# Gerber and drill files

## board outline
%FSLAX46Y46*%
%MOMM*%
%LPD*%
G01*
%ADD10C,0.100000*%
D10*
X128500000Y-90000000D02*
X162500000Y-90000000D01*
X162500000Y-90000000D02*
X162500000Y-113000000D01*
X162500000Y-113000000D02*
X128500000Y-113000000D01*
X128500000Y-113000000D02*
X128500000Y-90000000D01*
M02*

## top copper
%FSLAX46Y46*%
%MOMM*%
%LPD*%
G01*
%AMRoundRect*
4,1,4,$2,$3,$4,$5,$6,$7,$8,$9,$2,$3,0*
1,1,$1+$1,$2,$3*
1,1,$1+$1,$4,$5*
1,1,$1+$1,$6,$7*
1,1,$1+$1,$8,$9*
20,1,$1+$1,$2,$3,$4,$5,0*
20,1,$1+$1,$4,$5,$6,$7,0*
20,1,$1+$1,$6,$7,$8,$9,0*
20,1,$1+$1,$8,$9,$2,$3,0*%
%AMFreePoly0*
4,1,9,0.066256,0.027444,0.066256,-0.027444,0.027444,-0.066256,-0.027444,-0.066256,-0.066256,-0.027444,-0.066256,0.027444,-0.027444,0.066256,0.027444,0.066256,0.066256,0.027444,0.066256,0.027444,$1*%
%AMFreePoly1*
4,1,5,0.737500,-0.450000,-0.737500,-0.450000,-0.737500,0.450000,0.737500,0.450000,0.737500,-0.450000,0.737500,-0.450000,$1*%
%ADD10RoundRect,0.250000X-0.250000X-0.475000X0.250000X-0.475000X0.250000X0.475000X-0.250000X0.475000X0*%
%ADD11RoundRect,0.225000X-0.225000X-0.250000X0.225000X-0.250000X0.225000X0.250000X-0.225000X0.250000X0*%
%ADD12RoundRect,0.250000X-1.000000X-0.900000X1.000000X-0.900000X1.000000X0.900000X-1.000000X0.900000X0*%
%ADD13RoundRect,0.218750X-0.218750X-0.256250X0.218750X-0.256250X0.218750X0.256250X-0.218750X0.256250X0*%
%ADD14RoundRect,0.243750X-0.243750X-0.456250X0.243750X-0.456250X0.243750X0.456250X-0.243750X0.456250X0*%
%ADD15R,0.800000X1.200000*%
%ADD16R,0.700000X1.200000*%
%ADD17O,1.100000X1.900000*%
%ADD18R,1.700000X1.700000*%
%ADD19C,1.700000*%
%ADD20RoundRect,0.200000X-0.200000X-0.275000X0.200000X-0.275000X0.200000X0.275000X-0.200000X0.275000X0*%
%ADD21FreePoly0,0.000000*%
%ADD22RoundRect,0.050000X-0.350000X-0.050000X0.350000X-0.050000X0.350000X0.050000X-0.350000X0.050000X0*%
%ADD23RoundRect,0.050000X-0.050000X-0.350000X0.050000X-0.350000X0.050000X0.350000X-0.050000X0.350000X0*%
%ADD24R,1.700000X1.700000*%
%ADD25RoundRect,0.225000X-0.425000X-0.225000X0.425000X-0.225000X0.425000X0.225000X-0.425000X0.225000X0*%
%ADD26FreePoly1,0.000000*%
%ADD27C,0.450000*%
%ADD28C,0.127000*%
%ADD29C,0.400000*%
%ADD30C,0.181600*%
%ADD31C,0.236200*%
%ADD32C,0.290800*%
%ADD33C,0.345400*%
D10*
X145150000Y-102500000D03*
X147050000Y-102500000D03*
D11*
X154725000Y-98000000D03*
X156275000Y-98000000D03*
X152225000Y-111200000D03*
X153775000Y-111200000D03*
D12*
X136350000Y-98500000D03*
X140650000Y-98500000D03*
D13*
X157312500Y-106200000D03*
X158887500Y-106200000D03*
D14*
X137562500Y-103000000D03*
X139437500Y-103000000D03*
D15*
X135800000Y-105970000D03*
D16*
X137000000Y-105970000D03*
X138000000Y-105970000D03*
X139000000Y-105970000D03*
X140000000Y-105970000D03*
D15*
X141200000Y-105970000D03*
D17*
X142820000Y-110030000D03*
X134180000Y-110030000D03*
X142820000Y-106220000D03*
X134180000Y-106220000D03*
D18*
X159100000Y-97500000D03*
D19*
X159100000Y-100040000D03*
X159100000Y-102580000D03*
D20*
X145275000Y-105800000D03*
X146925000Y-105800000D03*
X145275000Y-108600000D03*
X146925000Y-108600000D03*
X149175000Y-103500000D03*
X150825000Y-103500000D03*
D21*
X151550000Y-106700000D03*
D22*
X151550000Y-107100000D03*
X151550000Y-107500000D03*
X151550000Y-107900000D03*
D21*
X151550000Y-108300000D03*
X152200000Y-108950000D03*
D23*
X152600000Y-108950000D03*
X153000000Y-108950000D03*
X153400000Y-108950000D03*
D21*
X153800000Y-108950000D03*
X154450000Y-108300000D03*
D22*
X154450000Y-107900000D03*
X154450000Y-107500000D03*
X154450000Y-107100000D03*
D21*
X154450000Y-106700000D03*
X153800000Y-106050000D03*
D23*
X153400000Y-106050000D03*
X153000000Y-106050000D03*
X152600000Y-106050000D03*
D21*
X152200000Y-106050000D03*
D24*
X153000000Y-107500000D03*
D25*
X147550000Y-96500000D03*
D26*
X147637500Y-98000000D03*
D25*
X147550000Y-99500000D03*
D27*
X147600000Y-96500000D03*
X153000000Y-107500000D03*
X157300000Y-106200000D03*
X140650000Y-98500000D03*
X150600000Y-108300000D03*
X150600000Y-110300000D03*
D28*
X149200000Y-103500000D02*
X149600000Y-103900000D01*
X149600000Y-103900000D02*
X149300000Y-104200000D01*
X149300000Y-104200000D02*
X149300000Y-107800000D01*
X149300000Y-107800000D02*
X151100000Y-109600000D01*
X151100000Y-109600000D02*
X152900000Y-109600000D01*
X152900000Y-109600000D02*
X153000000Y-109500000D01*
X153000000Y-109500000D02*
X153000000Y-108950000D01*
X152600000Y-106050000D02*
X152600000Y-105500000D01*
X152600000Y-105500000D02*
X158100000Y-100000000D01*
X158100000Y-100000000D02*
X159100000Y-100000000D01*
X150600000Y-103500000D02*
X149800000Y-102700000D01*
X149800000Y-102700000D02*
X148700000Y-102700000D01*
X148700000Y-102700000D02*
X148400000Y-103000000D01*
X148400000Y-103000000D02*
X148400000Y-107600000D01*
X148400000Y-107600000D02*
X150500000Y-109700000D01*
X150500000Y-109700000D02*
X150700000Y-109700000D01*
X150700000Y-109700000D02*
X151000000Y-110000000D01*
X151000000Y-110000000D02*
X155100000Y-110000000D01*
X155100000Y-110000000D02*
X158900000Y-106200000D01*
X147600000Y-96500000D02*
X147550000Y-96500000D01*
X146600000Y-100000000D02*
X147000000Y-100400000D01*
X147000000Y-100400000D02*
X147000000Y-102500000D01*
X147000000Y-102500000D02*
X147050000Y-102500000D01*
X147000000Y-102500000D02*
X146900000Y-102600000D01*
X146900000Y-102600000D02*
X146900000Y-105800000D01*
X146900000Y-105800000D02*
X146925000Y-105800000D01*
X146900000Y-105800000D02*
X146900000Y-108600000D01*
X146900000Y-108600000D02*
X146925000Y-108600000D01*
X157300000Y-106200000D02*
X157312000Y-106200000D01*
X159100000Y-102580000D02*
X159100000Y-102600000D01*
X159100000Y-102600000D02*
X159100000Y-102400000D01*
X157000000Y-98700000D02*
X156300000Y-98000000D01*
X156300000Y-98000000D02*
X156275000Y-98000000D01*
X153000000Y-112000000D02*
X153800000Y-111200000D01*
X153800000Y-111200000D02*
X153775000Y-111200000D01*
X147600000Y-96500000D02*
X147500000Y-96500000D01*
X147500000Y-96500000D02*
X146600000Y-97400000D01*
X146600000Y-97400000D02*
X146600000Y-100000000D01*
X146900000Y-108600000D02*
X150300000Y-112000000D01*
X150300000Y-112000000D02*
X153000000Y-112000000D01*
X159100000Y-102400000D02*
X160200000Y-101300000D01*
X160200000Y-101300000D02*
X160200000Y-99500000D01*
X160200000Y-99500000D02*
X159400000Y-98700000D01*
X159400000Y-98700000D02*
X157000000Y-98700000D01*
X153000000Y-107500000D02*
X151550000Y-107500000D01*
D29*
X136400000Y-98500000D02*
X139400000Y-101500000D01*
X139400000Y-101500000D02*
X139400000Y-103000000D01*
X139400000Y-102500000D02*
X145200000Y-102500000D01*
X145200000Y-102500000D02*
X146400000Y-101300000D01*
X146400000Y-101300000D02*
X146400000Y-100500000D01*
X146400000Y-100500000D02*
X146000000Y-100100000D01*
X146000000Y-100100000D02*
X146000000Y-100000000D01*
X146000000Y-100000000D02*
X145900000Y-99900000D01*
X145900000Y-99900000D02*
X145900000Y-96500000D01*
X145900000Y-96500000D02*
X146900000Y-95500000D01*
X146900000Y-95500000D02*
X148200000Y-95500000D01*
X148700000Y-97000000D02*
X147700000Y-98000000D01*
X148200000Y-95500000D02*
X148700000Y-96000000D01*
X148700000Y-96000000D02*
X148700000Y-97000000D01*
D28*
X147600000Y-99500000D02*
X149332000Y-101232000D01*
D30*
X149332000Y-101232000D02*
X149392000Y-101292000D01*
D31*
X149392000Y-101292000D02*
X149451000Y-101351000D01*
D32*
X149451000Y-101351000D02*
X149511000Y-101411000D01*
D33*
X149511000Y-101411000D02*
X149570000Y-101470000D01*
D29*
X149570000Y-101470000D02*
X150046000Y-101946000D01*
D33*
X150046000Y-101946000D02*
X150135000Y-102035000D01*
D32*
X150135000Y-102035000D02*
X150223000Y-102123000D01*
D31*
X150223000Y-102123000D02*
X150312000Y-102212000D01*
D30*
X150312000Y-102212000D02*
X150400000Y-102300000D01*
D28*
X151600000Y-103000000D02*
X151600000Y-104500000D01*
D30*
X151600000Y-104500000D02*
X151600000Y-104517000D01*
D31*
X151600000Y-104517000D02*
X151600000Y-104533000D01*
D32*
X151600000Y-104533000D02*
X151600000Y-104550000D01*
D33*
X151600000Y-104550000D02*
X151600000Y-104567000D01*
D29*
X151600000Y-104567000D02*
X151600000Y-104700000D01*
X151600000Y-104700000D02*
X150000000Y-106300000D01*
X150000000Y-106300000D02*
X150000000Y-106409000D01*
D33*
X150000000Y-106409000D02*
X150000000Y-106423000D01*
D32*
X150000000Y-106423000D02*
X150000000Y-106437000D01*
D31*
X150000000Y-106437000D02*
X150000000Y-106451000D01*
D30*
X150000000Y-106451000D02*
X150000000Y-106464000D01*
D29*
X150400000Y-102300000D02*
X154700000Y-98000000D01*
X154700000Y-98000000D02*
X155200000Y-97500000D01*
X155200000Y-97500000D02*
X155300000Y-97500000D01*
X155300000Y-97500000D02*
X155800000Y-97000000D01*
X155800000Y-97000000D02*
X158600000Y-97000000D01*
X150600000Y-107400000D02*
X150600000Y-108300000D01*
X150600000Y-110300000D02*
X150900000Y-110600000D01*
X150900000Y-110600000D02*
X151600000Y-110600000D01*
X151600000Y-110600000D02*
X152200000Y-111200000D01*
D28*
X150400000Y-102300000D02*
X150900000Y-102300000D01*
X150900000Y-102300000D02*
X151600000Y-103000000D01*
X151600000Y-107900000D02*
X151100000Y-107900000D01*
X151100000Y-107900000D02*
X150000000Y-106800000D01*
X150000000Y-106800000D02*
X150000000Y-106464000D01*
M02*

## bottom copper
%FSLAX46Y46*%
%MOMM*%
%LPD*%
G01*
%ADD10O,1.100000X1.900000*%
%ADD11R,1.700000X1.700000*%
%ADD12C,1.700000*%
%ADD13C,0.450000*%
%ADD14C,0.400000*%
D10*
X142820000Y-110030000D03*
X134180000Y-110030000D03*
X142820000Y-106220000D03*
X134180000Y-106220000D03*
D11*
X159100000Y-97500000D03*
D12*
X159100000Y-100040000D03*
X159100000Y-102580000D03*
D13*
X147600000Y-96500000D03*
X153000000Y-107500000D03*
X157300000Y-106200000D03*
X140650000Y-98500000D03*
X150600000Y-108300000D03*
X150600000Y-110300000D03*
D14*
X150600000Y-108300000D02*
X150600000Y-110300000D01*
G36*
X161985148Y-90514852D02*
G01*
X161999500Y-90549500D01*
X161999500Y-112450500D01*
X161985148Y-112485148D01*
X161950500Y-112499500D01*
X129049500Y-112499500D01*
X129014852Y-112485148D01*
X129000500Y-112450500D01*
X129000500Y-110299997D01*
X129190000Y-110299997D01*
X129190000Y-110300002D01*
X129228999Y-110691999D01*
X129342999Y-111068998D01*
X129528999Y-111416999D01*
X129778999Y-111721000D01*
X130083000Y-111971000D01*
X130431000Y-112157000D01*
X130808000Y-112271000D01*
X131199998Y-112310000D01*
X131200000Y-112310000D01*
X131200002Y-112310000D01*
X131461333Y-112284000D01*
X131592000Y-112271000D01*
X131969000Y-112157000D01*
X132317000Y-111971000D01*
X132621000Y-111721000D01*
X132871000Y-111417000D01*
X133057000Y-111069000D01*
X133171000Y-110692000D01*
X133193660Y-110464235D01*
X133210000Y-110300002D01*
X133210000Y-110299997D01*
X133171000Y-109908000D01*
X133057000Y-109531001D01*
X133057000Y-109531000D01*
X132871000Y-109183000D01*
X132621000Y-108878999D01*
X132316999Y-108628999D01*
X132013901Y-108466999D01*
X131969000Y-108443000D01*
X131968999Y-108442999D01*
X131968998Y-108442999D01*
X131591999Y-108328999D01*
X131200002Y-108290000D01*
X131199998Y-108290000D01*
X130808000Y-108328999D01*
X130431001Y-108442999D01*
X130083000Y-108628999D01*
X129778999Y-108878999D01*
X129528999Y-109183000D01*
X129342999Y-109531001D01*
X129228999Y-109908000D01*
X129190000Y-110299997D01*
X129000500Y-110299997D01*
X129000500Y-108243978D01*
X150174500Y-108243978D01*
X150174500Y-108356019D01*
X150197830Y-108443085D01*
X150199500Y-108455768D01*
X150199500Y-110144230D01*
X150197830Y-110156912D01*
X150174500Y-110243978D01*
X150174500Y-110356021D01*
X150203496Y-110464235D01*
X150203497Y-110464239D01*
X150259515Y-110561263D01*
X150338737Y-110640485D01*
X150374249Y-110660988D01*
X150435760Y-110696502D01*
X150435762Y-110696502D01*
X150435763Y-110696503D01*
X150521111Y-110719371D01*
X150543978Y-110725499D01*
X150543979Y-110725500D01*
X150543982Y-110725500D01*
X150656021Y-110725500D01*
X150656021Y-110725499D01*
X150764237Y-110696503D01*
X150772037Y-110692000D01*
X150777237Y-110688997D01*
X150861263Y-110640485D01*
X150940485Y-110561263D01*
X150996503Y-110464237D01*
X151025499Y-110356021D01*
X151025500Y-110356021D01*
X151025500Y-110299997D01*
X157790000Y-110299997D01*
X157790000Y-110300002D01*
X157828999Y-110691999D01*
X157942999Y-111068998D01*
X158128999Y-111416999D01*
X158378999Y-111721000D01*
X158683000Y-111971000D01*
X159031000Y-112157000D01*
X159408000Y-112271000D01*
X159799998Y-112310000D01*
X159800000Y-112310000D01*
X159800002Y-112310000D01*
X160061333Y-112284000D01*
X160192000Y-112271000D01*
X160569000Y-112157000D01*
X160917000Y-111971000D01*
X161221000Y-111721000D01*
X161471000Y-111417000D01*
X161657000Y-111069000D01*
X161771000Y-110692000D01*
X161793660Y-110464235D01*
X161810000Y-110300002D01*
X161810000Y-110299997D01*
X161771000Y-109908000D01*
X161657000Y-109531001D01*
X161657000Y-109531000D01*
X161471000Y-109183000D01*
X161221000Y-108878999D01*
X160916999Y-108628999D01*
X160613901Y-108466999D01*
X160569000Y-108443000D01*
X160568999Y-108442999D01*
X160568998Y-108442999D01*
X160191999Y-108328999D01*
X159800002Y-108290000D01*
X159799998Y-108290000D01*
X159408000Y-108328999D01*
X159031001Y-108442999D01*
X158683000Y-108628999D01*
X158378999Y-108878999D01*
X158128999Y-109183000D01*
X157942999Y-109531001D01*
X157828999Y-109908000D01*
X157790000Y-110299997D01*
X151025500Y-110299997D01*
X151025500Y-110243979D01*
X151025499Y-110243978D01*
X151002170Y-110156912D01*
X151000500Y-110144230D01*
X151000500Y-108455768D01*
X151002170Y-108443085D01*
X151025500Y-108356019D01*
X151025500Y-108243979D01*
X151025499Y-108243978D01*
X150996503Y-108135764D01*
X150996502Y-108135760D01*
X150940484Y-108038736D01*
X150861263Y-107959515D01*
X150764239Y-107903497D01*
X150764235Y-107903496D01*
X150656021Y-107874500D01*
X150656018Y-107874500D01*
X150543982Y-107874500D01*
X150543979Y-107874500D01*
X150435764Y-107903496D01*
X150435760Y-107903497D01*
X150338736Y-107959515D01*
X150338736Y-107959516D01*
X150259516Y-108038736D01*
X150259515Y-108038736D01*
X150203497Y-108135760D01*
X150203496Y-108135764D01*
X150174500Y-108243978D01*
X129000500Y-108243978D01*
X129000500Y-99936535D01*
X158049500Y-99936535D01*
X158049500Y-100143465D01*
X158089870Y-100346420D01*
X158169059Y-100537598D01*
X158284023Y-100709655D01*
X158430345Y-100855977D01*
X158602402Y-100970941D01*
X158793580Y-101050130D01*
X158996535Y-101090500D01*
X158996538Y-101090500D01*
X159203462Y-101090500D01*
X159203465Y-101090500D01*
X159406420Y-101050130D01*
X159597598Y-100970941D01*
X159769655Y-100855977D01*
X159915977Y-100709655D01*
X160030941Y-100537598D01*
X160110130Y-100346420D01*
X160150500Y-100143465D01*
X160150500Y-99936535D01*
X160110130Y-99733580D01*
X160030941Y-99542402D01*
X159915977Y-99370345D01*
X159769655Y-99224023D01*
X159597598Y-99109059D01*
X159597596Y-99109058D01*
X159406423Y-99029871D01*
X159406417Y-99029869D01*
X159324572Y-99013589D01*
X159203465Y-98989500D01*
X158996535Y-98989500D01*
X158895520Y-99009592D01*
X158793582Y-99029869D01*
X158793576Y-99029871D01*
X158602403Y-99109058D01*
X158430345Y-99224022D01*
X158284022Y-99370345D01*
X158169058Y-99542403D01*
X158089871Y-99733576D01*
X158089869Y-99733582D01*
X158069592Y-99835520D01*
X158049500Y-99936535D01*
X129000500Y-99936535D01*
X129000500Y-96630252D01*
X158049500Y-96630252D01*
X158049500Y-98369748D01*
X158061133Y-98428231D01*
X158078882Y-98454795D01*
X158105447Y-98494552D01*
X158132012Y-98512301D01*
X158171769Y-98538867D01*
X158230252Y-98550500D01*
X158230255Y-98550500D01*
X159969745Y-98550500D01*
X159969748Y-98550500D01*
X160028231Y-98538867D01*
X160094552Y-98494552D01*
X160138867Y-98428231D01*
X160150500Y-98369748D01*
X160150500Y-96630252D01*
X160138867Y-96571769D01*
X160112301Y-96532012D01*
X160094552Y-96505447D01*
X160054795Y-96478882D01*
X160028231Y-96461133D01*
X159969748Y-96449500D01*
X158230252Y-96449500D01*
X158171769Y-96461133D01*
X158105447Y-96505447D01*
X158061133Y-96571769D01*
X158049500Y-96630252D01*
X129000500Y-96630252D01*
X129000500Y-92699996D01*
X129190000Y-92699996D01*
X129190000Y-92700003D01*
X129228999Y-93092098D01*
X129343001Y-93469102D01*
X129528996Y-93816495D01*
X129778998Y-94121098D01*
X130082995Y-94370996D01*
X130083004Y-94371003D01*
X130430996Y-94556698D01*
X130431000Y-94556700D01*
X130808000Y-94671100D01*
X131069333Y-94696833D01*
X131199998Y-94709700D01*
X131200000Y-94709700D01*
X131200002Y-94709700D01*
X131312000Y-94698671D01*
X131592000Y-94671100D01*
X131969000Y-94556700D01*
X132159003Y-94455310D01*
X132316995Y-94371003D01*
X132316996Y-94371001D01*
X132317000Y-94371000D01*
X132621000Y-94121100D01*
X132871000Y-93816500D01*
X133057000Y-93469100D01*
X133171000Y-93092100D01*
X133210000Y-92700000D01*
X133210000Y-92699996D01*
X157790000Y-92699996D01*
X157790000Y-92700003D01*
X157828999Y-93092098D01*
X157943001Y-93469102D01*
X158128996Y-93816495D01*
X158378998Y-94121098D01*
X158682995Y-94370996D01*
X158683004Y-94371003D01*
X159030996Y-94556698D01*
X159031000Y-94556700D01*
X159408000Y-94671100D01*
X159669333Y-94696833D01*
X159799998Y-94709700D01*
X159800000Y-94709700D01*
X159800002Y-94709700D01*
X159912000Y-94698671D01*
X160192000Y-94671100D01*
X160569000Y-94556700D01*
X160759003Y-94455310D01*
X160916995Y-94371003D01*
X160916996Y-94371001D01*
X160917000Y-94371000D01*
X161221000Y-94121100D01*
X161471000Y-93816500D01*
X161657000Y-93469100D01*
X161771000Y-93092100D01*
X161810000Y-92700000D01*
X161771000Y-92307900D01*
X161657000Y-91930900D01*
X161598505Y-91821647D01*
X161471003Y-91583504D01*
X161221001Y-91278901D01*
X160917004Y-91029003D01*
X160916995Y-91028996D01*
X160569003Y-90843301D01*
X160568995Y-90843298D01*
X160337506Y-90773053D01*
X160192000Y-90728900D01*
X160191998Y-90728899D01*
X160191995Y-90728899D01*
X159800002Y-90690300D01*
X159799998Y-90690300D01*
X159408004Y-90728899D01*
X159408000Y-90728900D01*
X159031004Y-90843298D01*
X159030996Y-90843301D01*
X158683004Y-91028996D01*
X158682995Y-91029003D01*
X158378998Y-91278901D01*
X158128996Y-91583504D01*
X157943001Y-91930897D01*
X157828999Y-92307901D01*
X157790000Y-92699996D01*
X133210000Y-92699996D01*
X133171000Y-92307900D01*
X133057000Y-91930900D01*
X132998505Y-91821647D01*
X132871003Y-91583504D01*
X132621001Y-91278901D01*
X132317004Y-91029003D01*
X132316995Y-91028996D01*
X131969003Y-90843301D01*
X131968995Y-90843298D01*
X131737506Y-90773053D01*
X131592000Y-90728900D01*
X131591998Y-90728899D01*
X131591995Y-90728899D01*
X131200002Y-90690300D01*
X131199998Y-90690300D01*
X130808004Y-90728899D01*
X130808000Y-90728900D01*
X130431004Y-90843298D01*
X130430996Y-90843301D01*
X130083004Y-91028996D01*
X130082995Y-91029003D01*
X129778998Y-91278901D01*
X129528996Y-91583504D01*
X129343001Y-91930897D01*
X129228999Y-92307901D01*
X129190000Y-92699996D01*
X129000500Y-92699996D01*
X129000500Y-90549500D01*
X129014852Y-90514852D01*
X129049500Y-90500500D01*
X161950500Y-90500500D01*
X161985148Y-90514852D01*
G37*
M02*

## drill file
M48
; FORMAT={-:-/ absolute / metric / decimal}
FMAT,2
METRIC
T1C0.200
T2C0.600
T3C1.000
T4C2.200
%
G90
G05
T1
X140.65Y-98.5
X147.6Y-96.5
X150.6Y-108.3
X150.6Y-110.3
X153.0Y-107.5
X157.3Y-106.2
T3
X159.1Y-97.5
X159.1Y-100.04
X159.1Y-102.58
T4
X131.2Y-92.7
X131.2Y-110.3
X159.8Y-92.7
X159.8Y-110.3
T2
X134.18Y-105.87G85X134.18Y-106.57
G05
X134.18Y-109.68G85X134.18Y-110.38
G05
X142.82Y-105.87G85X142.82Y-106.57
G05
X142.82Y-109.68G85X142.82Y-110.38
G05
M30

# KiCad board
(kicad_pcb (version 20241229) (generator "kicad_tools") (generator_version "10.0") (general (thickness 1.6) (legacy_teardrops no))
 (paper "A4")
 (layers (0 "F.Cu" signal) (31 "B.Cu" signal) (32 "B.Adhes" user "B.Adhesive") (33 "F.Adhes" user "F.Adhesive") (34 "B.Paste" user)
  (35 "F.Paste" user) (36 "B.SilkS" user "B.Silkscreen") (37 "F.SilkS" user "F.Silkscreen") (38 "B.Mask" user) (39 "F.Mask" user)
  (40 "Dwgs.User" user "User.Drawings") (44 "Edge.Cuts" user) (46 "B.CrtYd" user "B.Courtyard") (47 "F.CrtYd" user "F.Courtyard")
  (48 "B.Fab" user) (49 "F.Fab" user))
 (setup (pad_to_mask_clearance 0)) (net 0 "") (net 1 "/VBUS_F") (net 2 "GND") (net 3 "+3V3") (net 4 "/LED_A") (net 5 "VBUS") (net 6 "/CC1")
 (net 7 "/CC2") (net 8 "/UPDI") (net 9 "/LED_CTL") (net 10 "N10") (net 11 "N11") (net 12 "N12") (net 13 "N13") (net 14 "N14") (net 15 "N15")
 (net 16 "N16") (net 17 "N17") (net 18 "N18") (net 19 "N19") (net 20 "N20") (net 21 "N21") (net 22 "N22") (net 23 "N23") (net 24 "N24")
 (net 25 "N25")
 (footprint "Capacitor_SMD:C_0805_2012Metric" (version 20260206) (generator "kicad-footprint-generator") (layer "F.Cu") (at 146.1 102.5)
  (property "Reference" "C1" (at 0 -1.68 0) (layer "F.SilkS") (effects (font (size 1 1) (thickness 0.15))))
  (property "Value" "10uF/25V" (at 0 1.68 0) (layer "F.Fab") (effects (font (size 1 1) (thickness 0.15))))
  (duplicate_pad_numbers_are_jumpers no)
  (pad "1" smd roundrect (at -0.95 0) (size 1 1.45) (layers "F.Cu" "F.Mask" "F.Paste") (roundrect_rratio 0.25) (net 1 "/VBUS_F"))
  (pad "2" smd roundrect (at 0.95 0) (size 1 1.45) (layers "F.Cu" "F.Mask" "F.Paste") (roundrect_rratio 0.25) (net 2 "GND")))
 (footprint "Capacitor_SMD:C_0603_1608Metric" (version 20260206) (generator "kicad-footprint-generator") (layer "F.Cu") (at 155.5 98)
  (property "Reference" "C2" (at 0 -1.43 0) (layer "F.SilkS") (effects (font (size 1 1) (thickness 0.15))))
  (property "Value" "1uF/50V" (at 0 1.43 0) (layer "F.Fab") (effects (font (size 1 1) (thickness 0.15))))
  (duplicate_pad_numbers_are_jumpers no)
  (pad "1" smd roundrect (at -0.775 0) (size 0.9 0.95) (layers "F.Cu" "F.Mask" "F.Paste") (roundrect_rratio 0.25) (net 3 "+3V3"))
  (pad "2" smd roundrect (at 0.775 0) (size 0.9 0.95) (layers "F.Cu" "F.Mask" "F.Paste") (roundrect_rratio 0.25) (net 2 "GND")))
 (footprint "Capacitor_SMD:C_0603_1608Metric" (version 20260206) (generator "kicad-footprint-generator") (layer "F.Cu") (at 153 111.2)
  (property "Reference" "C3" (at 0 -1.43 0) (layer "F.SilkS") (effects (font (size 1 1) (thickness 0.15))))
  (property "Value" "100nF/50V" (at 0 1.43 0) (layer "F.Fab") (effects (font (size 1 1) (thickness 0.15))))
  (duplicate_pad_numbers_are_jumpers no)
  (pad "1" smd roundrect (at -0.775 0) (size 0.9 0.95) (layers "F.Cu" "F.Mask" "F.Paste") (roundrect_rratio 0.25) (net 3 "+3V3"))
  (pad "2" smd roundrect (at 0.775 0) (size 0.9 0.95) (layers "F.Cu" "F.Mask" "F.Paste") (roundrect_rratio 0.25) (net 2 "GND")))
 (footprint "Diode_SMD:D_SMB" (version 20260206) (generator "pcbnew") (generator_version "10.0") (layer "F.Cu") (at 138.5 98.5)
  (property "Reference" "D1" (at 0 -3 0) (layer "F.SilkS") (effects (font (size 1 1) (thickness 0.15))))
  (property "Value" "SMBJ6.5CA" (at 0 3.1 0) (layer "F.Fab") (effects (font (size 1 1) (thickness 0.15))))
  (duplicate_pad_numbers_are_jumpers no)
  (pad "1" smd roundrect (at -2.15 0) (size 2.5 2.3) (layers "F.Cu" "F.Mask" "F.Paste") (roundrect_rratio 0.1086956522) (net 1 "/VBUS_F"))
  (pad "2" smd roundrect (at 2.15 0) (size 2.5 2.3) (layers "F.Cu" "F.Mask" "F.Paste") (roundrect_rratio 0.1086956522) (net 2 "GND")))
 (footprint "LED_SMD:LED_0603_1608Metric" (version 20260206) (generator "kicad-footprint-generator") (layer "F.Cu") (at 158.1 106.2)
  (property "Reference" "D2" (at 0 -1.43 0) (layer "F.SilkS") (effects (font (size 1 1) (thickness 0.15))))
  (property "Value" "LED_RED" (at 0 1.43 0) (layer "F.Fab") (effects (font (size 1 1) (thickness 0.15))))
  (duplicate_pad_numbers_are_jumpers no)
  (pad "1" smd roundrect (at -0.7875 0) (size 0.875 0.95) (layers "F.Cu" "F.Mask" "F.Paste") (roundrect_rratio 0.25) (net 2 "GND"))
  (pad "2" smd roundrect (at 0.7875 0) (size 0.875 0.95) (layers "F.Cu" "F.Mask" "F.Paste") (roundrect_rratio 0.25) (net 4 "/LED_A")))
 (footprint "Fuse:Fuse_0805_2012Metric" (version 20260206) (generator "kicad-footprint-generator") (layer "F.Cu") (at 138.5 103)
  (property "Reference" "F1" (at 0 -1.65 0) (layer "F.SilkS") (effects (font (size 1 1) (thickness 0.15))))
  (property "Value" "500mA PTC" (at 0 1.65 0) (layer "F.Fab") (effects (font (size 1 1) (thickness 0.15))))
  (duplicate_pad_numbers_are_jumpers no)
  (pad "1" smd roundrect (at -0.9375 0) (size 0.975 1.4) (layers "F.Cu" "F.Mask" "F.Paste") (roundrect_rratio 0.25) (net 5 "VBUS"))
  (pad "2" smd roundrect (at 0.9375 0) (size 0.975 1.4) (layers "F.Cu" "F.Mask" "F.Paste") (roundrect_rratio 0.25) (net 1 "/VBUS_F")))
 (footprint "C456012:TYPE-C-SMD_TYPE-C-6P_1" (layer "F.Cu") (at 138.5 108)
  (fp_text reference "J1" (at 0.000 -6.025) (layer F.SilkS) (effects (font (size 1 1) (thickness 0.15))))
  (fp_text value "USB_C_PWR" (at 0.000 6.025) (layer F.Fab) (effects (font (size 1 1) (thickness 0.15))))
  (pad B12 smd rect (at -2.70 -2.03 0.00) (size 0.800 1.200) (layers F.Cu F.Paste F.Mask) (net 2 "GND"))
  (pad B9 smd rect (at -1.50 -2.03 0.00) (size 0.700 1.200) (layers F.Cu F.Paste F.Mask) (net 5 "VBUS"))
  (pad A5 smd rect (at -0.50 -2.03 0.00) (size 0.700 1.200) (layers F.Cu F.Paste F.Mask) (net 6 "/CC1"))
  (pad B5 smd rect (at 0.50 -2.03 0.00) (size 0.700 1.200) (layers F.Cu F.Paste F.Mask) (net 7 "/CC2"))
  (pad A9 smd rect (at 1.50 -2.03 0.00) (size 0.700 1.200) (layers F.Cu F.Paste F.Mask) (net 5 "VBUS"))
  (pad A12 smd rect (at 2.70 -2.03 0.00) (size 0.800 1.200) (layers F.Cu F.Paste F.Mask) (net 2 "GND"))
  (pad 7 thru_hole oval (at 4.32 2.03 0.00) (size 1.100 1.900) (layers *.Cu *.Mask) (drill oval 0.599998 1.299997) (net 2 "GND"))
  (pad 7 thru_hole oval (at -4.32 2.03 0.00) (size 1.100 1.900) (layers *.Cu *.Mask) (drill oval 0.599998 1.299997) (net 2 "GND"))
  (pad 7 thru_hole oval (at 4.32 -1.78 0.00) (size 1.100 1.900) (layers *.Cu *.Mask) (drill oval 0.599998 1.299997) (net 2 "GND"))
  (pad 7 thru_hole oval (at -4.32 -1.78 0.00) (size 1.100 1.900) (layers *.Cu *.Mask) (drill oval 0.599998 1.299997) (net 2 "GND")))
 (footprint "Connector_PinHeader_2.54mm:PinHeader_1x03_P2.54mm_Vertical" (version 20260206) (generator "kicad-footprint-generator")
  (layer "F.Cu") (at 159.1 97.5)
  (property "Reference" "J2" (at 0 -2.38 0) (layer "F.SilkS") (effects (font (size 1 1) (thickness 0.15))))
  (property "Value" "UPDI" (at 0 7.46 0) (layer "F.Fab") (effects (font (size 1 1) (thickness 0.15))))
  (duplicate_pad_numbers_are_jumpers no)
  (pad "1" thru_hole rect (at 0 0) (size 1.7 1.7) (drill 1) (layers "*.Cu" "*.Mask") (remove_unused_layers no) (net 3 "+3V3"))
  (pad "2" thru_hole circle (at 0 2.54) (size 1.7 1.7) (drill 1) (layers "*.Cu" "*.Mask") (remove_unused_layers no) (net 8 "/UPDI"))
  (pad "3" thru_hole circle (at 0 5.08) (size 1.7 1.7) (drill 1) (layers "*.Cu" "*.Mask") (remove_unused_layers no) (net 2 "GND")))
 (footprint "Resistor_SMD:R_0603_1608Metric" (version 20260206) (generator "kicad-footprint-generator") (layer "F.Cu") (at 146.1 105.8)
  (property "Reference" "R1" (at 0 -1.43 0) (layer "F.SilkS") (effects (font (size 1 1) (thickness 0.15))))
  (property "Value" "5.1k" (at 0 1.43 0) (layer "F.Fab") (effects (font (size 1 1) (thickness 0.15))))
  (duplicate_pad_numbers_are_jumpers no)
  (pad "1" smd roundrect (at -0.825 0) (size 0.8 0.95) (layers "F.Cu" "F.Mask" "F.Paste") (roundrect_rratio 0.25) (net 6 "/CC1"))
  (pad "2" smd roundrect (at 0.825 0) (size 0.8 0.95) (layers "F.Cu" "F.Mask" "F.Paste") (roundrect_rratio 0.25) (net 2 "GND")))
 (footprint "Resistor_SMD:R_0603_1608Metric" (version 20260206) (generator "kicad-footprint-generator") (layer "F.Cu") (at 146.1 108.6)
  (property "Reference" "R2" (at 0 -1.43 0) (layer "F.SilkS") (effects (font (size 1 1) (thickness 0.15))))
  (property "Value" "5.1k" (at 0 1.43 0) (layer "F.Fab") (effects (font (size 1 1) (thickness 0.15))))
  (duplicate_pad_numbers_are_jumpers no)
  (pad "1" smd roundrect (at -0.825 0) (size 0.8 0.95) (layers "F.Cu" "F.Mask" "F.Paste") (roundrect_rratio 0.25) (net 7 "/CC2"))
  (pad "2" smd roundrect (at 0.825 0) (size 0.8 0.95) (layers "F.Cu" "F.Mask" "F.Paste") (roundrect_rratio 0.25) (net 2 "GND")))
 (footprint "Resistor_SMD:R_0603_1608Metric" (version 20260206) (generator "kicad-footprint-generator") (layer "F.Cu") (at 150 103.5)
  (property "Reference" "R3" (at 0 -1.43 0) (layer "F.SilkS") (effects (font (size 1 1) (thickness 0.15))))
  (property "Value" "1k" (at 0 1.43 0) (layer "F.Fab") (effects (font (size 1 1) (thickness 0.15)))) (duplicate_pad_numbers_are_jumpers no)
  (pad "1" smd roundrect (at -0.825 0) (size 0.8 0.95) (layers "F.Cu" "F.Mask" "F.Paste") (roundrect_rratio 0.25) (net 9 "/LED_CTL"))
  (pad "2" smd roundrect (at 0.825 0) (size 0.8 0.95) (layers "F.Cu" "F.Mask" "F.Paste") (roundrect_rratio 0.25) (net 4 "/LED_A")))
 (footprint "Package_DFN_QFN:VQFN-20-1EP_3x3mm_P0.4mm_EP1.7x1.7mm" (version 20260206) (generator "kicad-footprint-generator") (layer "F.Cu")
  (at 153 107.5)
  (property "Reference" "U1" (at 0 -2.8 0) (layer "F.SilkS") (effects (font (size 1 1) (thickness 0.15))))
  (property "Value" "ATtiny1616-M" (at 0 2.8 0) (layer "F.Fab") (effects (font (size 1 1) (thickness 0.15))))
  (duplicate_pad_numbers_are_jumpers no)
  (pad "" smd roundrect (at -0.425 -0.425) (size 0.69 0.69) (layers "F.Paste") (roundrect_rratio 0.25))
  (pad "" smd roundrect (at -0.425 0.425) (size 0.69 0.69) (layers "F.Paste") (roundrect_rratio 0.25))
  (pad "" smd roundrect (at 0.425 -0.425) (size 0.69 0.69) (layers "F.Paste") (roundrect_rratio 0.25))
  (pad "" smd roundrect (at 0.425 0.425) (size 0.69 0.69) (layers "F.Paste") (roundrect_rratio 0.25))
  (pad "1" smd custom (at -1.45 -0.8) (size 0.143431 0.143431) (layers "F.Cu" "F.Mask" "F.Paste")
   (options (clearance outline) (anchor circle)) (primitives) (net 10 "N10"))
  (pad "2" smd roundrect (at -1.45 -0.4) (size 0.8 0.2) (layers "F.Cu" "F.Mask" "F.Paste") (roundrect_rratio 0.25) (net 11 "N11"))
  (pad "3" smd roundrect (at -1.45 0) (size 0.8 0.2) (layers "F.Cu" "F.Mask" "F.Paste") (roundrect_rratio 0.25) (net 2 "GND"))
  (pad "4" smd roundrect (at -1.45 0.4) (size 0.8 0.2) (layers "F.Cu" "F.Mask" "F.Paste") (roundrect_rratio 0.25) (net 3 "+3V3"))
  (pad "5" smd custom (at -1.45 0.8) (size 0.143431 0.143431) (layers "F.Cu" "F.Mask" "F.Paste")
   (options (clearance outline) (anchor circle)) (primitives) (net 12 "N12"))
  (pad "6" smd custom (at -0.8 1.45) (size 0.143431 0.143431) (layers "F.Cu" "F.Mask" "F.Paste")
   (options (clearance outline) (anchor circle)) (primitives) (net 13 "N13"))
  (pad "7" smd roundrect (at -0.4 1.45) (size 0.2 0.8) (layers "F.Cu" "F.Mask" "F.Paste") (roundrect_rratio 0.25) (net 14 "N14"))
  (pad "8" smd roundrect (at 0 1.45) (size 0.2 0.8) (layers "F.Cu" "F.Mask" "F.Paste") (roundrect_rratio 0.25) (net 9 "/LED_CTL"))
  (pad "9" smd roundrect (at 0.4 1.45) (size 0.2 0.8) (layers "F.Cu" "F.Mask" "F.Paste") (roundrect_rratio 0.25) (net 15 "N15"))
  (pad "10" smd custom (at 0.8 1.45) (size 0.143431 0.143431) (layers "F.Cu" "F.Mask" "F.Paste")
   (options (clearance outline) (anchor circle)) (primitives) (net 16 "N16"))
  (pad "11" smd custom (at 1.45 0.8) (size 0.143431 0.143431) (layers "F.Cu" "F.Mask" "F.Paste")
   (options (clearance outline) (anchor circle)) (primitives) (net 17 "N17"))
  (pad "12" smd roundrect (at 1.45 0.4) (size 0.8 0.2) (layers "F.Cu" "F.Mask" "F.Paste") (roundrect_rratio 0.25) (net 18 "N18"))
  (pad "13" smd roundrect (at 1.45 0) (size 0.8 0.2) (layers "F.Cu" "F.Mask" "F.Paste") (roundrect_rratio 0.25) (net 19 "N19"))
  (pad "14" smd roundrect (at 1.45 -0.4) (size 0.8 0.2) (layers "F.Cu" "F.Mask" "F.Paste") (roundrect_rratio 0.25) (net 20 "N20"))
  (pad "15" smd custom (at 1.45 -0.8) (size 0.143431 0.143431) (layers "F.Cu" "F.Mask" "F.Paste")
   (options (clearance outline) (anchor circle)) (primitives) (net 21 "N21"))
  (pad "16" smd custom (at 0.8 -1.45) (size 0.143431 0.143431) (layers "F.Cu" "F.Mask" "F.Paste")
   (options (clearance outline) (anchor circle)) (primitives) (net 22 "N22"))
  (pad "17" smd roundrect (at 0.4 -1.45) (size 0.2 0.8) (layers "F.Cu" "F.Mask" "F.Paste") (roundrect_rratio 0.25) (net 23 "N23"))
  (pad "18" smd roundrect (at 0 -1.45) (size 0.2 0.8) (layers "F.Cu" "F.Mask" "F.Paste") (roundrect_rratio 0.25) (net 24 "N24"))
  (pad "19" smd roundrect (at -0.4 -1.45) (size 0.2 0.8) (layers "F.Cu" "F.Mask" "F.Paste") (roundrect_rratio 0.25) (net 8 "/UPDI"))
  (pad "20" smd custom (at -0.8 -1.45) (size 0.143431 0.143431) (layers "F.Cu" "F.Mask" "F.Paste")
   (options (clearance outline) (anchor circle)) (primitives) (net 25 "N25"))
  (pad "21" smd rect (at 0 0) (size 1.7 1.7) (layers "F.Cu" "F.Mask") (zone_connect 2) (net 2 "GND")))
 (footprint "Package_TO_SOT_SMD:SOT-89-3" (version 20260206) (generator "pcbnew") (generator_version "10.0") (layer "F.Cu") (at 149.5 98)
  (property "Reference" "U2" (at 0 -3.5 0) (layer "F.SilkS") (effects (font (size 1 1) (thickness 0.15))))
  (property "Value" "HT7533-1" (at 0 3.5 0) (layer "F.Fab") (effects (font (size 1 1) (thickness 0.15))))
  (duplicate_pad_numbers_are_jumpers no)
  (pad "1" smd roundrect (at -1.95 -1.5) (size 1.3 0.9) (layers "F.Cu" "F.Mask" "F.Paste") (roundrect_rratio 0.25) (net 2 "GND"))
  (pad "2" smd custom (at -1.8625 0) (size 1.475 0.9) (layers "F.Cu" "F.Mask" "F.Paste") (zone_connect 2) (thermal_bridge_angle 45)
   (options (clearance outline) (anchor rect)) (primitives) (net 1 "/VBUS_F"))
  (pad "3" smd roundrect (at -1.95 1.5) (size 1.3 0.9) (layers "F.Cu" "F.Mask" "F.Paste") (roundrect_rratio 0.25) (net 3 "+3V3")))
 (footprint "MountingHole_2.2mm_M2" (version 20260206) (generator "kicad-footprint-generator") (layer "F.Cu") (at 131.2 92.7)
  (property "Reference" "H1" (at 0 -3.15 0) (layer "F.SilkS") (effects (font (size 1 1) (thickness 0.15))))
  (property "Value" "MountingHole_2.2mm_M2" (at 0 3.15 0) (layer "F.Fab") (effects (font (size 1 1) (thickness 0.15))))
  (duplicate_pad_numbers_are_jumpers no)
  (pad "" np_thru_hole circle (at 0 0) (size 2.2 2.2) (drill 2.2) (layers "*.Cu" "*.Mask")))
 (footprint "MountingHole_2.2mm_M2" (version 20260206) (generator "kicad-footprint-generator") (layer "F.Cu") (at 159.8 92.7)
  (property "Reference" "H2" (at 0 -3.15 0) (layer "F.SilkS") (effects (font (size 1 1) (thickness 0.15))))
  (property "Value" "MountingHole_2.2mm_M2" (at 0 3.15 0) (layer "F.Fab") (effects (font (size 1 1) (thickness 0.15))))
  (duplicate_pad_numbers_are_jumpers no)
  (pad "" np_thru_hole circle (at 0 0) (size 2.2 2.2) (drill 2.2) (layers "*.Cu" "*.Mask")))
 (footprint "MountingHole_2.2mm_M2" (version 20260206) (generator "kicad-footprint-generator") (layer "F.Cu") (at 131.2 110.3)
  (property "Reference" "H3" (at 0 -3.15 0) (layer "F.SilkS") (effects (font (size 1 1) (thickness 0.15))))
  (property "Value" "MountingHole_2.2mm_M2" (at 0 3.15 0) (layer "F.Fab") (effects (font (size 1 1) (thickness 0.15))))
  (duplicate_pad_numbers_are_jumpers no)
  (pad "" np_thru_hole circle (at 0 0) (size 2.2 2.2) (drill 2.2) (layers "*.Cu" "*.Mask")))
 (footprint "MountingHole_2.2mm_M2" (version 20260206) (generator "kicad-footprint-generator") (layer "F.Cu") (at 159.8 110.3)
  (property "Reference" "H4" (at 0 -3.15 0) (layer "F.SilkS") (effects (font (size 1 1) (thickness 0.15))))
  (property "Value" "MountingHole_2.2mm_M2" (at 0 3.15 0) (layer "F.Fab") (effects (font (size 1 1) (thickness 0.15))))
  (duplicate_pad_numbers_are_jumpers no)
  (pad "" np_thru_hole circle (at 0 0) (size 2.2 2.2) (drill 2.2) (layers "*.Cu" "*.Mask")))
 (gr_line (start 128.5 90) (end 162.5 90) (stroke (width 0.1) (type default)) (layer "Edge.Cuts"))
 (gr_line (start 162.5 90) (end 162.5 113) (stroke (width 0.1) (type default)) (layer "Edge.Cuts"))
 (gr_line (start 162.5 113) (end 128.5 113) (stroke (width 0.1) (type default)) (layer "Edge.Cuts"))
 (gr_line (start 128.5 113) (end 128.5 90) (stroke (width 0.1) (type default)) (layer "Edge.Cuts"))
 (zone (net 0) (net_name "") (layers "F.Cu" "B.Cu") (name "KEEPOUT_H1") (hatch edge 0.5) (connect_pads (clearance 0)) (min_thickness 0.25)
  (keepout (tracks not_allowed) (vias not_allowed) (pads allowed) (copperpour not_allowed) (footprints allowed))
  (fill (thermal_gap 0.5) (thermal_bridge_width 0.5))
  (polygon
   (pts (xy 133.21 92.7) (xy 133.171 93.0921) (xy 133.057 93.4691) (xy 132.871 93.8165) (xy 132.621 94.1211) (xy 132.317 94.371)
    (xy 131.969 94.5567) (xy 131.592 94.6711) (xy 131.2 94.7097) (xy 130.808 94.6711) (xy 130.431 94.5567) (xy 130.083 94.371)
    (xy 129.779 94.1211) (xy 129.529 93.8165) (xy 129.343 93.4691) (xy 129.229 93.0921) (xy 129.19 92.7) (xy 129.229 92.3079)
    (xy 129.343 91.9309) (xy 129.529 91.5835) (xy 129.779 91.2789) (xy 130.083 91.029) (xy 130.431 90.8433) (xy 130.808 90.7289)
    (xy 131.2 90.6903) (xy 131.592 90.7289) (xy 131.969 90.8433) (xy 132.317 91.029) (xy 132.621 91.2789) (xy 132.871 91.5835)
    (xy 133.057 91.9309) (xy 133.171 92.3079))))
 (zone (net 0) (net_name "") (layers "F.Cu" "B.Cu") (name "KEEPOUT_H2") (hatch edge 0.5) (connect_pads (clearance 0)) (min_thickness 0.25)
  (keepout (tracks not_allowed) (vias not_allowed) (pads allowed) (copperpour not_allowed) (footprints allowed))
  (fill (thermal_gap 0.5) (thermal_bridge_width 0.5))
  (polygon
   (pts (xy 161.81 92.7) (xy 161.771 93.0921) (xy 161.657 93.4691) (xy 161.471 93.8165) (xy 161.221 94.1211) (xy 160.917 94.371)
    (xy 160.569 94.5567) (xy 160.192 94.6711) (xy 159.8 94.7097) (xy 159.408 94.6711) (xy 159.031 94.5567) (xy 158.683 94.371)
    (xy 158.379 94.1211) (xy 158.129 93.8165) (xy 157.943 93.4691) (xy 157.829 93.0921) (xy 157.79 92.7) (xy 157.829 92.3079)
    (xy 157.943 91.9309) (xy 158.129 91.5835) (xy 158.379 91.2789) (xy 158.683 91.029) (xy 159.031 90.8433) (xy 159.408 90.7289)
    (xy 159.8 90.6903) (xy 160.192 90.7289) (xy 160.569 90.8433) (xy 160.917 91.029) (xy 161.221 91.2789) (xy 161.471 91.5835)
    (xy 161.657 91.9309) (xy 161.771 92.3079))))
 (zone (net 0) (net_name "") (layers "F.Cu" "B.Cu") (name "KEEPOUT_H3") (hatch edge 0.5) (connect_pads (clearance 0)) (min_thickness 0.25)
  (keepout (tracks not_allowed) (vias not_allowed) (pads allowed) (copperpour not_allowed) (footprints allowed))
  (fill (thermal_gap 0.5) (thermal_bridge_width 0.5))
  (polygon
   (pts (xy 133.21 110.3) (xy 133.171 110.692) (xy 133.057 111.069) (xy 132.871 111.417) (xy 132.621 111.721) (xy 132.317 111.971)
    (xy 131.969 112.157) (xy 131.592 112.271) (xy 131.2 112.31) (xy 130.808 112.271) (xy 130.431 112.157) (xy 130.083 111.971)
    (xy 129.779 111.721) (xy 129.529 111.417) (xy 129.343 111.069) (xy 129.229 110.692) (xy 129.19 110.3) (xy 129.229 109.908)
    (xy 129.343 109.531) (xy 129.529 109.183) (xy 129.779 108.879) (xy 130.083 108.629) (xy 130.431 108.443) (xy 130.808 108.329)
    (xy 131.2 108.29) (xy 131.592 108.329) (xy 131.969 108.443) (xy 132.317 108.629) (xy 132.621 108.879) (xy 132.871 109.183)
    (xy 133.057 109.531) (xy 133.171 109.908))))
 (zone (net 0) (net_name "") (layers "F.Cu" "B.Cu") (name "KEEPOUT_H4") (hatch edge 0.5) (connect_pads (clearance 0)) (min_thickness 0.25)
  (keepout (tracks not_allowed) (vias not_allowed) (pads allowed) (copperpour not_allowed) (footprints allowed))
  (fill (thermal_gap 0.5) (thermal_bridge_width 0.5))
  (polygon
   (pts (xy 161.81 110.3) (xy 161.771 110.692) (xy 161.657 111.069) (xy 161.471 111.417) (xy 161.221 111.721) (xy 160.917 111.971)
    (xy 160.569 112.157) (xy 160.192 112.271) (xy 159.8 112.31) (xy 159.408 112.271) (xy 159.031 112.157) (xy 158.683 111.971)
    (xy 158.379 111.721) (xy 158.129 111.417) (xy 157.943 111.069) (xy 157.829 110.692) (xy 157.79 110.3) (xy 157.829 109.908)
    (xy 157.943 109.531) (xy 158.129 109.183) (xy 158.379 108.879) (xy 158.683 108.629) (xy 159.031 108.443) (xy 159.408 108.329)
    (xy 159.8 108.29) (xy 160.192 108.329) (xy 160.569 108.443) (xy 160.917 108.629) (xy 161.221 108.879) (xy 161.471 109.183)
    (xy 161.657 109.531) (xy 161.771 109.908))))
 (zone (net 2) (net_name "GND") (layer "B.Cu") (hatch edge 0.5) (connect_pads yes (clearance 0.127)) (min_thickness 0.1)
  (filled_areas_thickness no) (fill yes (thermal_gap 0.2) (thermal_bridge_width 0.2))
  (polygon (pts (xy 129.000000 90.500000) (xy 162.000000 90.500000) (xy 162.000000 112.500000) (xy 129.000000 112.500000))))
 (segment (start 149.2 103.5) (end 149.6 103.9) (width 0.127) (layer "F.Cu") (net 9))
 (segment (start 149.6 103.9) (end 149.3 104.2) (width 0.127) (layer "F.Cu") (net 9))
 (segment (start 149.3 104.2) (end 149.3 107.8) (width 0.127) (layer "F.Cu") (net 9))
 (segment (start 149.3 107.8) (end 151.1 109.6) (width 0.127) (layer "F.Cu") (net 9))
 (segment (start 151.1 109.6) (end 152.9 109.6) (width 0.127) (layer "F.Cu") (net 9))
 (segment (start 152.9 109.6) (end 153 109.5) (width 0.127) (layer "F.Cu") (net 9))
 (segment (start 153 109.5) (end 153 108.95) (width 0.127) (layer "F.Cu") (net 9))
 (segment (start 152.6 106.05) (end 152.6 105.5) (width 0.127) (layer "F.Cu") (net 8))
 (segment (start 152.6 105.5) (end 158.1 100) (width 0.127) (layer "F.Cu") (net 8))
 (segment (start 158.1 100) (end 159.1 100) (width 0.127) (layer "F.Cu") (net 8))
 (segment (start 150.6 103.5) (end 149.8 102.7) (width 0.127) (layer "F.Cu") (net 4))
 (segment (start 149.8 102.7) (end 148.7 102.7) (width 0.127) (layer "F.Cu") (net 4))
 (segment (start 148.7 102.7) (end 148.4 103) (width 0.127) (layer "F.Cu") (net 4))
 (segment (start 148.4 103) (end 148.4 107.6) (width 0.127) (layer "F.Cu") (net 4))
 (segment (start 148.4 107.6) (end 150.5 109.7) (width 0.127) (layer "F.Cu") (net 4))
 (segment (start 150.5 109.7) (end 150.7 109.7) (width 0.127) (layer "F.Cu") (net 4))
 (segment (start 150.7 109.7) (end 151 110) (width 0.127) (layer "F.Cu") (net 4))
 (segment (start 151 110) (end 155.1 110) (width 0.127) (layer "F.Cu") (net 4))
 (segment (start 155.1 110) (end 158.9 106.2) (width 0.127) (layer "F.Cu") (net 4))
 (segment (start 147.6 96.5) (end 147.55 96.5) (width 0.127) (layer "F.Cu") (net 2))
 (segment (start 146.6 100) (end 147 100.4) (width 0.127) (layer "F.Cu") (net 2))
 (segment (start 147 100.4) (end 147 102.5) (width 0.127) (layer "F.Cu") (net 2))
 (segment (start 147 102.5) (end 147.05 102.5) (width 0.127) (layer "F.Cu") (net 2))
 (segment (start 147 102.5) (end 146.9 102.6) (width 0.127) (layer "F.Cu") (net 2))
 (segment (start 146.9 102.6) (end 146.9 105.8) (width 0.127) (layer "F.Cu") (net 2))
 (segment (start 146.9 105.8) (end 146.925 105.8) (width 0.127) (layer "F.Cu") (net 2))
 (segment (start 146.9 105.8) (end 146.9 108.6) (width 0.127) (layer "F.Cu") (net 2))
 (segment (start 146.9 108.6) (end 146.925 108.6) (width 0.127) (layer "F.Cu") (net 2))
 (segment (start 157.3 106.2) (end 157.312 106.2) (width 0.127) (layer "F.Cu") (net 2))
 (segment (start 159.1 102.58) (end 159.1 102.6) (width 0.127) (layer "F.Cu") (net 2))
 (segment (start 159.1 102.6) (end 159.1 102.4) (width 0.127) (layer "F.Cu") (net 2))
 (segment (start 157 98.7) (end 156.3 98) (width 0.127) (layer "F.Cu") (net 2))
 (segment (start 156.3 98) (end 156.275 98) (width 0.127) (layer "F.Cu") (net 2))
 (segment (start 153 112) (end 153.8 111.2) (width 0.127) (layer "F.Cu") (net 2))
 (segment (start 153.8 111.2) (end 153.775 111.2) (width 0.127) (layer "F.Cu") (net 2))
 (segment (start 147.6 96.5) (end 147.5 96.5) (width 0.127) (layer "F.Cu") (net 2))
 (segment (start 147.5 96.5) (end 146.6 97.4) (width 0.127) (layer "F.Cu") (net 2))
 (segment (start 146.6 97.4) (end 146.6 100) (width 0.127) (layer "F.Cu") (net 2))
 (segment (start 146.9 108.6) (end 150.3 112) (width 0.127) (layer "F.Cu") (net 2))
 (segment (start 150.3 112) (end 153 112) (width 0.127) (layer "F.Cu") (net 2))
 (segment (start 159.1 102.4) (end 160.2 101.3) (width 0.127) (layer "F.Cu") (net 2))
 (segment (start 160.2 101.3) (end 160.2 99.5) (width 0.127) (layer "F.Cu") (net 2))
 (segment (start 160.2 99.5) (end 159.4 98.7) (width 0.127) (layer "F.Cu") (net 2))
 (segment (start 159.4 98.7) (end 157 98.7) (width 0.127) (layer "F.Cu") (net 2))
 (segment (start 153 107.5) (end 151.55 107.5) (width 0.127) (layer "F.Cu") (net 2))
 (segment (start 136.4 98.5) (end 139.4 101.5) (width 0.4) (layer "F.Cu") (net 1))
 (segment (start 139.4 101.5) (end 139.4 103) (width 0.4) (layer "F.Cu") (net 1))
 (segment (start 139.4 102.5) (end 145.2 102.5) (width 0.4) (layer "F.Cu") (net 1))
 (segment (start 145.2 102.5) (end 146.4 101.3) (width 0.4) (layer "F.Cu") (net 1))
 (segment (start 146.4 101.3) (end 146.4 100.5) (width 0.4) (layer "F.Cu") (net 1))
 (segment (start 146.4 100.5) (end 146 100.1) (width 0.4) (layer "F.Cu") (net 1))
 (segment (start 146 100.1) (end 146 100) (width 0.4) (layer "F.Cu") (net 1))
 (segment (start 146 100) (end 145.9 99.9) (width 0.4) (layer "F.Cu") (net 1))
 (segment (start 145.9 99.9) (end 145.9 96.5) (width 0.4) (layer "F.Cu") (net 1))
 (segment (start 145.9 96.5) (end 146.9 95.5) (width 0.4) (layer "F.Cu") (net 1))
 (segment (start 146.9 95.5) (end 148.2 95.5) (width 0.4) (layer "F.Cu") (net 1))
 (segment (start 148.7 97) (end 147.7 98) (width 0.4) (layer "F.Cu") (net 1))
 (segment (start 148.2 95.5) (end 148.7 96) (width 0.4) (layer "F.Cu") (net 1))
 (segment (start 148.7 96) (end 148.7 97) (width 0.4) (layer "F.Cu") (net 1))
 (segment (start 147.6 99.5) (end 149.332 101.232) (width 0.127) (layer "F.Cu") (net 3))
 (segment (start 149.332 101.232) (end 149.392 101.292) (width 0.1816) (layer "F.Cu") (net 3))
 (segment (start 149.392 101.292) (end 149.451 101.351) (width 0.2362) (layer "F.Cu") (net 3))
 (segment (start 149.451 101.351) (end 149.511 101.411) (width 0.2908) (layer "F.Cu") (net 3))
 (segment (start 149.511 101.411) (end 149.57 101.47) (width 0.3454) (layer "F.Cu") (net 3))
 (segment (start 149.57 101.47) (end 150.046 101.946) (width 0.4) (layer "F.Cu") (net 3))
 (segment (start 150.046 101.946) (end 150.135 102.035) (width 0.3454) (layer "F.Cu") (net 3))
 (segment (start 150.135 102.035) (end 150.223 102.123) (width 0.2908) (layer "F.Cu") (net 3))
 (segment (start 150.223 102.123) (end 150.312 102.212) (width 0.2362) (layer "F.Cu") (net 3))
 (segment (start 150.312 102.212) (end 150.4 102.3) (width 0.1816) (layer "F.Cu") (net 3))
 (segment (start 151.6 103) (end 151.6 104.5) (width 0.127) (layer "F.Cu") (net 3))
 (segment (start 151.6 104.5) (end 151.6 104.517) (width 0.1816) (layer "F.Cu") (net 3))
 (segment (start 151.6 104.517) (end 151.6 104.533) (width 0.2362) (layer "F.Cu") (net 3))
 (segment (start 151.6 104.533) (end 151.6 104.55) (width 0.2908) (layer "F.Cu") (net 3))
 (segment (start 151.6 104.55) (end 151.6 104.567) (width 0.3454) (layer "F.Cu") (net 3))
 (segment (start 151.6 104.567) (end 151.6 104.7) (width 0.4) (layer "F.Cu") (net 3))
 (segment (start 151.6 104.7) (end 150 106.3) (width 0.4) (layer "F.Cu") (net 3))
 (segment (start 150 106.3) (end 150 106.409) (width 0.4) (layer "F.Cu") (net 3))
 (segment (start 150 106.409) (end 150 106.423) (width 0.3454) (layer "F.Cu") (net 3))
 (segment (start 150 106.423) (end 150 106.437) (width 0.2908) (layer "F.Cu") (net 3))
 (segment (start 150 106.437) (end 150 106.451) (width 0.2362) (layer "F.Cu") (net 3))
 (segment (start 150 106.451) (end 150 106.464) (width 0.1816) (layer "F.Cu") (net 3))
 (segment (start 150.4 102.3) (end 154.7 98) (width 0.4) (layer "F.Cu") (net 3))
 (segment (start 154.7 98) (end 155.2 97.5) (width 0.4) (layer "F.Cu") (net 3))
 (segment (start 155.2 97.5) (end 155.3 97.5) (width 0.4) (layer "F.Cu") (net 3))
 (segment (start 155.3 97.5) (end 155.8 97) (width 0.4) (layer "F.Cu") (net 3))
 (segment (start 155.8 97) (end 158.6 97) (width 0.4) (layer "F.Cu") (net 3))
 (segment (start 150.6 107.4) (end 150.6 108.3) (width 0.4) (layer "F.Cu") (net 3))
 (segment (start 150.6 108.3) (end 150.6 110.3) (width 0.4) (layer "B.Cu") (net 3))
 (segment (start 150.6 110.3) (end 150.9 110.6) (width 0.4) (layer "F.Cu") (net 3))
 (segment (start 150.9 110.6) (end 151.6 110.6) (width 0.4) (layer "F.Cu") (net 3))
 (segment (start 151.6 110.6) (end 152.2 111.2) (width 0.4) (layer "F.Cu") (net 3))
 (segment (start 150.4 102.3) (end 150.9 102.3) (width 0.127) (layer "F.Cu") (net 3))
 (segment (start 150.9 102.3) (end 151.6 103) (width 0.127) (layer "F.Cu") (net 3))
 (segment (start 151.6 107.9) (end 151.1 107.9) (width 0.127) (layer "F.Cu") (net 3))
 (segment (start 151.1 107.9) (end 150 106.8) (width 0.127) (layer "F.Cu") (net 3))
 (segment (start 150 106.8) (end 150 106.464) (width 0.127) (layer "F.Cu") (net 3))
 (via (at 147.6 96.5) (size 0.45) (drill 0.2) (layers "F.Cu" "B.Cu") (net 2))
 (via (at 153 107.5) (size 0.45) (drill 0.2) (layers "F.Cu" "B.Cu") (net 2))
 (via (at 157.3 106.2) (size 0.45) (drill 0.2) (layers "F.Cu" "B.Cu") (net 2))
 (via (at 140.65 98.5) (size 0.45) (drill 0.2) (layers "F.Cu" "B.Cu") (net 2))
 (via (at 150.6 108.3) (size 0.45) (drill 0.2) (layers "F.Cu" "B.Cu") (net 3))
 (via (at 150.6 110.3) (size 0.45) (drill 0.2) (layers "F.Cu" "B.Cu") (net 3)))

